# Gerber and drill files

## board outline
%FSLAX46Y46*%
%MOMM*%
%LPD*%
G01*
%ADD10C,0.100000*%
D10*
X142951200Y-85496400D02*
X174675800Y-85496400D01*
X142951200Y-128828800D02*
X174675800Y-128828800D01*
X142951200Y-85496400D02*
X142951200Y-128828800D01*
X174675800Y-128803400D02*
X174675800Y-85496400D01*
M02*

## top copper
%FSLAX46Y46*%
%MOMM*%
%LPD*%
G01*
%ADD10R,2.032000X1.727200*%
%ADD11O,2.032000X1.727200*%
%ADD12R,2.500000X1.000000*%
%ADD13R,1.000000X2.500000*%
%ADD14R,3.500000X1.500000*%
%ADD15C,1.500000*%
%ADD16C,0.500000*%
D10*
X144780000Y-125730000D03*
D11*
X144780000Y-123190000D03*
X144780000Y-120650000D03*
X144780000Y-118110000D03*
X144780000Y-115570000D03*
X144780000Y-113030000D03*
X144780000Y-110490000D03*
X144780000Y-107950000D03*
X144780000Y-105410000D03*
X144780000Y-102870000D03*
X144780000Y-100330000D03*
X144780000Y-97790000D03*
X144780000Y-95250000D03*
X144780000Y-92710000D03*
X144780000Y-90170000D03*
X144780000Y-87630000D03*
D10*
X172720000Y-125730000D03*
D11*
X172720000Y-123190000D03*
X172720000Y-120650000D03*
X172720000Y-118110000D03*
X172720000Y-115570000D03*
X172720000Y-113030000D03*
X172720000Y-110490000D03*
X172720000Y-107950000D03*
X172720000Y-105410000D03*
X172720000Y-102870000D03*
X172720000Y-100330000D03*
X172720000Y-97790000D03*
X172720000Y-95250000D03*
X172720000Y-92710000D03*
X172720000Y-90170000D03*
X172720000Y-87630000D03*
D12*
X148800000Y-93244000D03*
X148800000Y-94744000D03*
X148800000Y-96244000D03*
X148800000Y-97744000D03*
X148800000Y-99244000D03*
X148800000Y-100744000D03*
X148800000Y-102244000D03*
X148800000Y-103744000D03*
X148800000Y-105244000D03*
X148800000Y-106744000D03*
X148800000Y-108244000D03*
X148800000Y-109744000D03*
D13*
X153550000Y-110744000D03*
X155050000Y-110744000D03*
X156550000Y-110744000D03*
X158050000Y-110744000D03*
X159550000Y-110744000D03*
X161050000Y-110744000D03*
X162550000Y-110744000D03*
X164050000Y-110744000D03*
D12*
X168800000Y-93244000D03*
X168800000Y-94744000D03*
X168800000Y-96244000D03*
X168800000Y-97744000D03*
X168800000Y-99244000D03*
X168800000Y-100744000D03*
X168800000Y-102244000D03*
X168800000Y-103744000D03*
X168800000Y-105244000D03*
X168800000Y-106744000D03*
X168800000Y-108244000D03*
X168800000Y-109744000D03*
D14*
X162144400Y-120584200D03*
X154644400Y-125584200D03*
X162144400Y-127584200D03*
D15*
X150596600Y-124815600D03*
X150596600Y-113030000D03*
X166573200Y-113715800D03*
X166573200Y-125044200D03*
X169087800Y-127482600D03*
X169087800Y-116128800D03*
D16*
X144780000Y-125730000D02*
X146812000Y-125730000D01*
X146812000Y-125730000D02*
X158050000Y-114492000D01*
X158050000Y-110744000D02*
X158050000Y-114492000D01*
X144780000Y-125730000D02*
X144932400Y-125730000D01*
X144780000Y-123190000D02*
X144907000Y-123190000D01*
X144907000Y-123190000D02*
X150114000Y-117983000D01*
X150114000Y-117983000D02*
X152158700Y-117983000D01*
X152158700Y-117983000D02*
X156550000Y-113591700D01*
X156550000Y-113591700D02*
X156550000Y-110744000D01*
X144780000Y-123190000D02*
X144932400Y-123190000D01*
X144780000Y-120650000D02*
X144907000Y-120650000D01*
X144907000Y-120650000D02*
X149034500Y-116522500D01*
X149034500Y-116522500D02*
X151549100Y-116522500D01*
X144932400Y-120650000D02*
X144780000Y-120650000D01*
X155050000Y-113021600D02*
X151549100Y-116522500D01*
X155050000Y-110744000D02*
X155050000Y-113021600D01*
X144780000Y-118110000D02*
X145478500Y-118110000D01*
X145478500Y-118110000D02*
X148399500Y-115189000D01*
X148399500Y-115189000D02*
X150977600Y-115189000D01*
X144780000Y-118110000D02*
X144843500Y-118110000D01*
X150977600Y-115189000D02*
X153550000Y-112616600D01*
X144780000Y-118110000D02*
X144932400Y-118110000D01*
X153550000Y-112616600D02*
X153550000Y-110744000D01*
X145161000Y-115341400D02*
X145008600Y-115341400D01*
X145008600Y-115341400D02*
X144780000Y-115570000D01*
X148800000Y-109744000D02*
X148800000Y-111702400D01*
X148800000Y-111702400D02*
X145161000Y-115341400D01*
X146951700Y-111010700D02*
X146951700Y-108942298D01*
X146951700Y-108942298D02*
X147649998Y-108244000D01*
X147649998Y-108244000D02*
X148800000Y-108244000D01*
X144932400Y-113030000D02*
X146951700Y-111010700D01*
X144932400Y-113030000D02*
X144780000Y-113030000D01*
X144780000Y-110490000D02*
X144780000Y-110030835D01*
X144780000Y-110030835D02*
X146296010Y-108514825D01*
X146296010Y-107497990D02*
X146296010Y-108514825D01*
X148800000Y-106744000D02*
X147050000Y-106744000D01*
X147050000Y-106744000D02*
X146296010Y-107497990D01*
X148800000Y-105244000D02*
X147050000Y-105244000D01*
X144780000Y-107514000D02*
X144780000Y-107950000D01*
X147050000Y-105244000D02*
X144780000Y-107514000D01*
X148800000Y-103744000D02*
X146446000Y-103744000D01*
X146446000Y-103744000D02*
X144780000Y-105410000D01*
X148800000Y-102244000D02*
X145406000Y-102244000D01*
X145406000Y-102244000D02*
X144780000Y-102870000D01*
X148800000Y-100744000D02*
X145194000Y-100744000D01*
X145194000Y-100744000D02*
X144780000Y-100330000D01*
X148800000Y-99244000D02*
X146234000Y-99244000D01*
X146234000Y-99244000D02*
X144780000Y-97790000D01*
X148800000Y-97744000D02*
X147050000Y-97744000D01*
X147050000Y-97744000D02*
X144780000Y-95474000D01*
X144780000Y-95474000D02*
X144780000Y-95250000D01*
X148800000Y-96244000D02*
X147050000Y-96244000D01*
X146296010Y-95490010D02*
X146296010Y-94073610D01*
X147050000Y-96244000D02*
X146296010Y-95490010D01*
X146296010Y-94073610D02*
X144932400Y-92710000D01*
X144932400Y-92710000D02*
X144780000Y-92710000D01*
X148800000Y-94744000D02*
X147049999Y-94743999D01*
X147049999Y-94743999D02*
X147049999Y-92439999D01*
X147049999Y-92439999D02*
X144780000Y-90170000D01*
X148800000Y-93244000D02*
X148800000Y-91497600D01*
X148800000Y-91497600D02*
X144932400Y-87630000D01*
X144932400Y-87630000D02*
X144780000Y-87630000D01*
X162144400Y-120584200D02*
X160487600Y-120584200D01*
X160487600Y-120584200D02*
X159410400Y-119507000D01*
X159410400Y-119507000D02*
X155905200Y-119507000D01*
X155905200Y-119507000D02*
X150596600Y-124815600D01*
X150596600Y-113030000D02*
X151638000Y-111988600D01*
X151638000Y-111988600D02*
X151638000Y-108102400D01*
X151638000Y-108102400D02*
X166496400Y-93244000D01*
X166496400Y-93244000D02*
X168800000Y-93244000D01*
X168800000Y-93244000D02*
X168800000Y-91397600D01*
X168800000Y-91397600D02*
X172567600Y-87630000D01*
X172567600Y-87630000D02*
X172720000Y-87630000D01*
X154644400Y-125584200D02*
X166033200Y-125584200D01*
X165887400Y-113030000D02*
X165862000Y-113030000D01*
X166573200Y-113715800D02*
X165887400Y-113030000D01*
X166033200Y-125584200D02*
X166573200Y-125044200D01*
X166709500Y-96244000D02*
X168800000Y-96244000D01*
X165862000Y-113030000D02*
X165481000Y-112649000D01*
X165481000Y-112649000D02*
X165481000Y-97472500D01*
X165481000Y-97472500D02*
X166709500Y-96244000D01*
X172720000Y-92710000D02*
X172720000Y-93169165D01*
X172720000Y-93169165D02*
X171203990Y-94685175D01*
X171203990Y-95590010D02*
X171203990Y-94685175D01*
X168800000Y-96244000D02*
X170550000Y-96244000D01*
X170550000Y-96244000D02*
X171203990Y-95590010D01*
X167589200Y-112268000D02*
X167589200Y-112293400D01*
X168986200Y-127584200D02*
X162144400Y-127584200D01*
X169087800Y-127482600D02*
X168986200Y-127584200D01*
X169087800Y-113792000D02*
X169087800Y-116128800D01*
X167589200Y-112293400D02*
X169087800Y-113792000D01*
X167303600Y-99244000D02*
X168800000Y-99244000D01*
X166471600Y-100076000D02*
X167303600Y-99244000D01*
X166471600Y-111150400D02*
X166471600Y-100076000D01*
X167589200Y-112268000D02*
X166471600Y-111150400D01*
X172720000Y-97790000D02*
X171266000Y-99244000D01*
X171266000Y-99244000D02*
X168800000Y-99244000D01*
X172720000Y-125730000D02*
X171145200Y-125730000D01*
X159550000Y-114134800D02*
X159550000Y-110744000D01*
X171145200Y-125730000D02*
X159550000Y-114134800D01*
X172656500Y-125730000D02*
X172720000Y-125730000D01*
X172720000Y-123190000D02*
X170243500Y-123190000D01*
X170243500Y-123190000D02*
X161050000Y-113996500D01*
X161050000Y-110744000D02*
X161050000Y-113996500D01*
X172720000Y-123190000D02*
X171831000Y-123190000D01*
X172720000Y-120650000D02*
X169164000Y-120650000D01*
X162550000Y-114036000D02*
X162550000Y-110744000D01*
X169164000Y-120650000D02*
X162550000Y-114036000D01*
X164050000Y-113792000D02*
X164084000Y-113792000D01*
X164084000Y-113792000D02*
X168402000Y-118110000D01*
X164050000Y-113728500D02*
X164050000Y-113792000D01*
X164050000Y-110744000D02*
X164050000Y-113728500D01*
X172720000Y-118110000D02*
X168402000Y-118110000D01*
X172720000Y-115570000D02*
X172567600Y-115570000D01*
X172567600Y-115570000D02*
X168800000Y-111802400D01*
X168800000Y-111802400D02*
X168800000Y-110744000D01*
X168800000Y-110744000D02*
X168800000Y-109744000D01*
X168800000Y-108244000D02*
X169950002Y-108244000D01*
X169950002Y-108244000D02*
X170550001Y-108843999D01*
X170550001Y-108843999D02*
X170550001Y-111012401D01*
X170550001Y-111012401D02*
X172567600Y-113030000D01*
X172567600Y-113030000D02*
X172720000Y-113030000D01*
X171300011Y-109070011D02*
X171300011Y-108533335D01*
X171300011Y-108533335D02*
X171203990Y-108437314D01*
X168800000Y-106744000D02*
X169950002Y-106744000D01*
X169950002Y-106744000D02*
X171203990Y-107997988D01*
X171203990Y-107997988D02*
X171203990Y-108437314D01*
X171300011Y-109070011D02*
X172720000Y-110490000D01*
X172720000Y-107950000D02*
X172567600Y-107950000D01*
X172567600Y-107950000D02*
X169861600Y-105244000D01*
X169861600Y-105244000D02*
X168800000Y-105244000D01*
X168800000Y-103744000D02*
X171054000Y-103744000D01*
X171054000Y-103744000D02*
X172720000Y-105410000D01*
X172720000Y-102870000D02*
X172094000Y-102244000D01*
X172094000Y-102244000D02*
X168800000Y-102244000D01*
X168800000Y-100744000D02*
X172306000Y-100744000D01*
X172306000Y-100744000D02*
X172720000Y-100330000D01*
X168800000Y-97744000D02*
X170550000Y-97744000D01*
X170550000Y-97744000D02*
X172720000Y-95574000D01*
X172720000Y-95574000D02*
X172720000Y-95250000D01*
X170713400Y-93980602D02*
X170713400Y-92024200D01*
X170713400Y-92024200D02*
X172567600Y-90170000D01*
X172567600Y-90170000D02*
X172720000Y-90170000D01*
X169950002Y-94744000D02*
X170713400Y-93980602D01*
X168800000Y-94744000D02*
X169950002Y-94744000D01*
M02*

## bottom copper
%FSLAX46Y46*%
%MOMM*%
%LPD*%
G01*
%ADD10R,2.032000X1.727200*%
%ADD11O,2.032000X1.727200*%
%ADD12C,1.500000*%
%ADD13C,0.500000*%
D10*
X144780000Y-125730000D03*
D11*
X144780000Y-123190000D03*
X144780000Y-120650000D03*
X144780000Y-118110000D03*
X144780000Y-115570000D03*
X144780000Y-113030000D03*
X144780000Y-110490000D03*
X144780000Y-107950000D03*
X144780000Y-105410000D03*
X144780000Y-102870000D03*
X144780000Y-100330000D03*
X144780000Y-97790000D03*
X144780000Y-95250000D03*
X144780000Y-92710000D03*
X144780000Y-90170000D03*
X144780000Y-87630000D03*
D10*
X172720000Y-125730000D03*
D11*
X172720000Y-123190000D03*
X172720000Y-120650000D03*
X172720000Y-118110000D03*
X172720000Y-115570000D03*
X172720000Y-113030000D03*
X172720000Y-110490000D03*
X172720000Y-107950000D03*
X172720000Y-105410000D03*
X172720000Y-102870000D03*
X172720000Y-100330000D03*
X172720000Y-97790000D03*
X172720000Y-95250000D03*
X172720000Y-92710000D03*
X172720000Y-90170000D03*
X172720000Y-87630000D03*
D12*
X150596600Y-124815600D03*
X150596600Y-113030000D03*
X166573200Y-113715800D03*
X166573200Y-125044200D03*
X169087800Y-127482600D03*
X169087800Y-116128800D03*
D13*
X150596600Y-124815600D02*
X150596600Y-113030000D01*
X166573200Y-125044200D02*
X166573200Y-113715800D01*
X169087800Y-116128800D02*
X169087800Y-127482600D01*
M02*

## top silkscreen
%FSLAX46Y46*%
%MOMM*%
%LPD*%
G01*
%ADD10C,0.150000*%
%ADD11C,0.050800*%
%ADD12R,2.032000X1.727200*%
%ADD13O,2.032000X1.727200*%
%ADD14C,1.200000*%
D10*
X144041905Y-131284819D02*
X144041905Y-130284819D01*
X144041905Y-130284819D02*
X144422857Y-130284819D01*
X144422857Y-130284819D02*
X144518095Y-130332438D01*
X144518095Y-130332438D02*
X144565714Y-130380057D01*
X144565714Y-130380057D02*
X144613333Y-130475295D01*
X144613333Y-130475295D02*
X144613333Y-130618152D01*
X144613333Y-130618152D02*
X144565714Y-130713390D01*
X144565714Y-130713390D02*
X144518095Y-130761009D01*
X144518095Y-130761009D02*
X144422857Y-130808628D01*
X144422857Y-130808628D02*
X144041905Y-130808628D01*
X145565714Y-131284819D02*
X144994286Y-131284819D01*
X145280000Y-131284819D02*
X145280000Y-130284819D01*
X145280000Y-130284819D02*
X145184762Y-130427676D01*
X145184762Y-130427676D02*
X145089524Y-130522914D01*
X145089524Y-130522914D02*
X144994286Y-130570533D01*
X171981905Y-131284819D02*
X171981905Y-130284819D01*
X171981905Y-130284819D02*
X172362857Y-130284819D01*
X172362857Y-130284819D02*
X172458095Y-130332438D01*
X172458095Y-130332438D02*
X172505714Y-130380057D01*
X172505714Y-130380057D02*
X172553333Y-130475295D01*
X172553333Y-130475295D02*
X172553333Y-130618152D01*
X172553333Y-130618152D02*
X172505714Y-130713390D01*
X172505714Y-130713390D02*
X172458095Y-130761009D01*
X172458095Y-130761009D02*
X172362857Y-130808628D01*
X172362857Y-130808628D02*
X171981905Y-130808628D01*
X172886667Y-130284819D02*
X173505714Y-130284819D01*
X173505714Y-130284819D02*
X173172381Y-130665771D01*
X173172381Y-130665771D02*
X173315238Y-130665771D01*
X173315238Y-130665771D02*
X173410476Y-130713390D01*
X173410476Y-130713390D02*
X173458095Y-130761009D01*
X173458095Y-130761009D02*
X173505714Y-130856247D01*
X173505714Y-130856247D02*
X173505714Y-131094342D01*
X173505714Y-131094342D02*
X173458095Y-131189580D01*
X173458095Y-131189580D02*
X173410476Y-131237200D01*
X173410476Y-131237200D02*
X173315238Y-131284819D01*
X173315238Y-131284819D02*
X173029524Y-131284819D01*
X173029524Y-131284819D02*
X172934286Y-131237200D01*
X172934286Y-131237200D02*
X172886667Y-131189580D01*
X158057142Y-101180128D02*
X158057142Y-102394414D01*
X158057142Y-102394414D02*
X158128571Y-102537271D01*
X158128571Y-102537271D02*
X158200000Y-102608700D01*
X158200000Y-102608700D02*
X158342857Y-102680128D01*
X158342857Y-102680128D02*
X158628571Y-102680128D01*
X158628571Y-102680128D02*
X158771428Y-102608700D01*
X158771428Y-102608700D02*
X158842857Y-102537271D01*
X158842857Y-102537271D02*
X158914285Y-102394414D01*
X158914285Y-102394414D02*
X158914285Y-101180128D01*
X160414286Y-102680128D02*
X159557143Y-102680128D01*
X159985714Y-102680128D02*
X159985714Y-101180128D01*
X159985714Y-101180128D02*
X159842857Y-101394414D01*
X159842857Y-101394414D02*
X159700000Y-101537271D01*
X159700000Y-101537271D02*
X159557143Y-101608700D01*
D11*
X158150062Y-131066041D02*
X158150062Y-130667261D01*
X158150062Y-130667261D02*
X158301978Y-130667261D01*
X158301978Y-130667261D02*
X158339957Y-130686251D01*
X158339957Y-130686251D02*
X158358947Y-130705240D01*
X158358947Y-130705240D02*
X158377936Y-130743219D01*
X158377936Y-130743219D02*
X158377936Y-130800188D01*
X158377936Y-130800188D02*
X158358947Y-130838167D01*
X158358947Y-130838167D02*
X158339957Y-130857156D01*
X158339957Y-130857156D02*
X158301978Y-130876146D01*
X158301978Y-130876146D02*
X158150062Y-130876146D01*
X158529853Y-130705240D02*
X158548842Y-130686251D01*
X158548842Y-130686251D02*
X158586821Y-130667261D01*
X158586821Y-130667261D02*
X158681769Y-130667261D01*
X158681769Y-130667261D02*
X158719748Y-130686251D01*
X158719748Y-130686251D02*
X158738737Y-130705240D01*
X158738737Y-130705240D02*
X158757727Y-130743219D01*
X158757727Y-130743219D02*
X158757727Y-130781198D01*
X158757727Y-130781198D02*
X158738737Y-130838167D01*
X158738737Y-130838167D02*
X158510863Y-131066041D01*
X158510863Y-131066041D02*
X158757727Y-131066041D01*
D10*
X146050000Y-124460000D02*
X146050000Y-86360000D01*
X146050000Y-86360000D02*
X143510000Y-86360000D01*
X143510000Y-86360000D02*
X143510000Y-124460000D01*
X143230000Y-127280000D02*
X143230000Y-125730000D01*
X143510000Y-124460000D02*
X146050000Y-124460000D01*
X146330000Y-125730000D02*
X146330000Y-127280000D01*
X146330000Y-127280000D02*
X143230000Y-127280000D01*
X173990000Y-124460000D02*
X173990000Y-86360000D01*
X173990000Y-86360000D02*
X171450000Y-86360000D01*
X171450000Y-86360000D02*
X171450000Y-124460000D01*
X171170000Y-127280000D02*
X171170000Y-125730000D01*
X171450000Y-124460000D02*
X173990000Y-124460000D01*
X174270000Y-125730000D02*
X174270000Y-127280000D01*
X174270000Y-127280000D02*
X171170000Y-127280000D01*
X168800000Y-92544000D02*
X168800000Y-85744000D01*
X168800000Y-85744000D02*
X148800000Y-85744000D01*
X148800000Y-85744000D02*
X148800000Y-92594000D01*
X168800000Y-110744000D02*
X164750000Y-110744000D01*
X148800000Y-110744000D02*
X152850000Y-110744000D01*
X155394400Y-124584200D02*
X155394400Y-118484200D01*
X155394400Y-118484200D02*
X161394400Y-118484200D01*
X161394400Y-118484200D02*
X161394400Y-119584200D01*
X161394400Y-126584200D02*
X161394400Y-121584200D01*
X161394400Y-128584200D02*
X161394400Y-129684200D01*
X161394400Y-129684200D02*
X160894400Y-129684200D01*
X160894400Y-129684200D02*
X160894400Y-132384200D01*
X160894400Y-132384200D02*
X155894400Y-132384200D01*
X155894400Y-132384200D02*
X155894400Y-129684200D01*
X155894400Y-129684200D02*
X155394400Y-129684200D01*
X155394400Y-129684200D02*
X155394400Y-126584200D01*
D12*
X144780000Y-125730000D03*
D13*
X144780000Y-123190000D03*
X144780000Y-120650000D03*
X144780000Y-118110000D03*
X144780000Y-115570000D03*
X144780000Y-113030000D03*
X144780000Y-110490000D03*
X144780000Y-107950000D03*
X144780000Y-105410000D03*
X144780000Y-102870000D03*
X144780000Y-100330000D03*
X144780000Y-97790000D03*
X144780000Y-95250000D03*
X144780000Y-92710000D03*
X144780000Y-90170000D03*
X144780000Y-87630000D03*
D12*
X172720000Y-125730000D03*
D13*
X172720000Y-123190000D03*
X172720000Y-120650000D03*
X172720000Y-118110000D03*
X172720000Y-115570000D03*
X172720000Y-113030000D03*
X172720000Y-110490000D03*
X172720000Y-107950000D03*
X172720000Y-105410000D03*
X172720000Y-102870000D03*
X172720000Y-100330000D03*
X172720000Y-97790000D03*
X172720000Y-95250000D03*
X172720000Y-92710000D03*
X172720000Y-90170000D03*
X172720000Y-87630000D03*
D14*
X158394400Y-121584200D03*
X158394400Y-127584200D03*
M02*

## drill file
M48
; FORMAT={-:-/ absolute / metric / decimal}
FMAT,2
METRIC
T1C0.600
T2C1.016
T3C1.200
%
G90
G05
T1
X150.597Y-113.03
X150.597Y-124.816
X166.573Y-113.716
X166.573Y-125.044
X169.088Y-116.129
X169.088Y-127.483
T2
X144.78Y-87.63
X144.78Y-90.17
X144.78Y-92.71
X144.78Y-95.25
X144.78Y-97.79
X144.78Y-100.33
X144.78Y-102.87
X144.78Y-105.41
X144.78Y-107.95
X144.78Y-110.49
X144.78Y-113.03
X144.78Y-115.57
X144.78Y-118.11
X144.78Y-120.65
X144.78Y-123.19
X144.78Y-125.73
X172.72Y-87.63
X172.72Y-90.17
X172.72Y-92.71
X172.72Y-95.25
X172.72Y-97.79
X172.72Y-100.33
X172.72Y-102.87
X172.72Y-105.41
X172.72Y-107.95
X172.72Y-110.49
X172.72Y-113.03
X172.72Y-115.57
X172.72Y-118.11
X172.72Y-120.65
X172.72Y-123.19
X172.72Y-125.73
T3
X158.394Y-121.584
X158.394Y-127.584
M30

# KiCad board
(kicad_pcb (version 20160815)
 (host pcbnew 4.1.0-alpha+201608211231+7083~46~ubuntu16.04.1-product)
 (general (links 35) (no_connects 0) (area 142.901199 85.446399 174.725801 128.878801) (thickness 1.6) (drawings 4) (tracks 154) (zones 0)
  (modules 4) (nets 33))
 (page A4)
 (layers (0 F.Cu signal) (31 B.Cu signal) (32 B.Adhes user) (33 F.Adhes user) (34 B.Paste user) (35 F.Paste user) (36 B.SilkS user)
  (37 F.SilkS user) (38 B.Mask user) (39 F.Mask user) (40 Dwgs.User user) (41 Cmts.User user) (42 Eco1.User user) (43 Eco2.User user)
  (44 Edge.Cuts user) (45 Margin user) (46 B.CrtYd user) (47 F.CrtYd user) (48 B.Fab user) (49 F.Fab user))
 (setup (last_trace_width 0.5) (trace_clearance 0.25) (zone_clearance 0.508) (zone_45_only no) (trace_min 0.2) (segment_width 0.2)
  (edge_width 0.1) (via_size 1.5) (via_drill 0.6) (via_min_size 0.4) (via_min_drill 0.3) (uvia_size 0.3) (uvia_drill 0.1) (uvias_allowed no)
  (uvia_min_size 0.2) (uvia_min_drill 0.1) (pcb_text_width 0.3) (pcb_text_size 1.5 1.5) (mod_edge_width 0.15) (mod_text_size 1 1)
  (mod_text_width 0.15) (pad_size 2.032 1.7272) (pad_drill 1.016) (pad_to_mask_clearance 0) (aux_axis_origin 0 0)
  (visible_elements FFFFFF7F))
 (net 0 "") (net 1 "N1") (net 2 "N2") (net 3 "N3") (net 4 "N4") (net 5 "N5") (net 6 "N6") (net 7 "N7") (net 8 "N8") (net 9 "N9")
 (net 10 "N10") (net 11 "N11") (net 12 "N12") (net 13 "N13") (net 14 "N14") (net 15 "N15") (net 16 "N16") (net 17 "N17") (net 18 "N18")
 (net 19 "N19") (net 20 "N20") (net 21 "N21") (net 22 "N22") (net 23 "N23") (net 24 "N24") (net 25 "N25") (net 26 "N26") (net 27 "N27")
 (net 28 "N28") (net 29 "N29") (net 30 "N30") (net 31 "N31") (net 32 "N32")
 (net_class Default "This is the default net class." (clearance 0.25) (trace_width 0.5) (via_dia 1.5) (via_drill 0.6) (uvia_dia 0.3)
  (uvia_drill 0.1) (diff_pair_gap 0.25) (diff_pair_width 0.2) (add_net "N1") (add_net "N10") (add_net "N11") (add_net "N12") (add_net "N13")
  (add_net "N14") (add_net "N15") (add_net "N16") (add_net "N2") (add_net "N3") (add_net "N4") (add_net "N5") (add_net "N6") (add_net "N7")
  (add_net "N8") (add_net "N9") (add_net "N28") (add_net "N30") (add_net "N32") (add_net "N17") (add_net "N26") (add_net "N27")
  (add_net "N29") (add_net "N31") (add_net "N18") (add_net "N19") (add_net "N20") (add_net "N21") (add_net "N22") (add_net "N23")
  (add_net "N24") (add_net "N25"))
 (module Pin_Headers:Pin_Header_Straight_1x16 (layer F.Cu) (at 144.78 125.73 180)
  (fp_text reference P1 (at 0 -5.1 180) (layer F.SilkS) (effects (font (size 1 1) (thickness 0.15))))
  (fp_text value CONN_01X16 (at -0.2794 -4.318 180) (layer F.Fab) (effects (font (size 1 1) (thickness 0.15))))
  (fp_line (start -1.27 1.27) (end -1.27 39.37) (layer F.SilkS) (width 0.15))
  (fp_line (start -1.27 39.37) (end 1.27 39.37) (layer F.SilkS) (width 0.15))
  (fp_line (start 1.27 39.37) (end 1.27 1.27) (layer F.SilkS) (width 0.15))
  (fp_line (start 1.55 -1.55) (end 1.55 0) (layer F.SilkS) (width 0.15))
  (fp_line (start 1.27 1.27) (end -1.27 1.27) (layer F.SilkS) (width 0.15))
  (fp_line (start -1.55 0) (end -1.55 -1.55) (layer F.SilkS) (width 0.15))
  (fp_line (start -1.55 -1.55) (end 1.55 -1.55) (layer F.SilkS) (width 0.15))
  (pad 1 thru_hole rect (at 0 0 180) (size 2.032 1.7272) (drill 1.016) (layers *.Cu *.Mask F.SilkS) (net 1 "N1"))
  (pad 2 thru_hole oval (at 0 2.54 180) (size 2.032 1.7272) (drill 1.016) (layers *.Cu *.Mask F.SilkS) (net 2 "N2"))
  (pad 3 thru_hole oval (at 0 5.08 180) (size 2.032 1.7272) (drill 1.016) (layers *.Cu *.Mask F.SilkS) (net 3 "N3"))
  (pad 4 thru_hole oval (at 0 7.62 180) (size 2.032 1.7272) (drill 1.016) (layers *.Cu *.Mask F.SilkS) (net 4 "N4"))
  (pad 5 thru_hole oval (at 0 10.16 180) (size 2.032 1.7272) (drill 1.016) (layers *.Cu *.Mask F.SilkS) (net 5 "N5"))
  (pad 6 thru_hole oval (at 0 12.7 180) (size 2.032 1.7272) (drill 1.016) (layers *.Cu *.Mask F.SilkS) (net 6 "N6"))
  (pad 7 thru_hole oval (at 0 15.24 180) (size 2.032 1.7272) (drill 1.016) (layers *.Cu *.Mask F.SilkS) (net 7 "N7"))
  (pad 8 thru_hole oval (at 0 17.78 180) (size 2.032 1.7272) (drill 1.016) (layers *.Cu *.Mask F.SilkS) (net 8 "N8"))
  (pad 9 thru_hole oval (at 0 20.32 180) (size 2.032 1.7272) (drill 1.016) (layers *.Cu *.Mask F.SilkS) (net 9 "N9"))
  (pad 10 thru_hole oval (at 0 22.86 180) (size 2.032 1.7272) (drill 1.016) (layers *.Cu *.Mask F.SilkS) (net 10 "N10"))
  (pad 11 thru_hole oval (at 0 25.4 180) (size 2.032 1.7272) (drill 1.016) (layers *.Cu *.Mask F.SilkS) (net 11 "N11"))
  (pad 12 thru_hole oval (at 0 27.94 180) (size 2.032 1.7272) (drill 1.016) (layers *.Cu *.Mask F.SilkS) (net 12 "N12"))
  (pad 13 thru_hole oval (at 0 30.48 180) (size 2.032 1.7272) (drill 1.016) (layers *.Cu *.Mask F.SilkS) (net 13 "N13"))
  (pad 14 thru_hole oval (at 0 33.02 180) (size 2.032 1.7272) (drill 1.016) (layers *.Cu *.Mask F.SilkS) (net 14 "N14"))
  (pad 15 thru_hole oval (at 0 35.56 180) (size 2.032 1.7272) (drill 1.016) (layers *.Cu *.Mask F.SilkS) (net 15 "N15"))
  (pad 16 thru_hole oval (at 0 38.1 180) (size 2.032 1.7272) (drill 1.016) (layers *.Cu *.Mask F.SilkS) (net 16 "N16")))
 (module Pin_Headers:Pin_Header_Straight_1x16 (layer F.Cu) (at 172.72 125.73 180)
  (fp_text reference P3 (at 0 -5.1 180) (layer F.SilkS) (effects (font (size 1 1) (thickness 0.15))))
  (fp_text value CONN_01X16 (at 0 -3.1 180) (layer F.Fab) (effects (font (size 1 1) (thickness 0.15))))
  (fp_line (start -1.27 1.27) (end -1.27 39.37) (layer F.SilkS) (width 0.15))
  (fp_line (start -1.27 39.37) (end 1.27 39.37) (layer F.SilkS) (width 0.15))
  (fp_line (start 1.27 39.37) (end 1.27 1.27) (layer F.SilkS) (width 0.15))
  (fp_line (start 1.55 -1.55) (end 1.55 0) (layer F.SilkS) (width 0.15))
  (fp_line (start 1.27 1.27) (end -1.27 1.27) (layer F.SilkS) (width 0.15))
  (fp_line (start -1.55 0) (end -1.55 -1.55) (layer F.SilkS) (width 0.15))
  (fp_line (start -1.55 -1.55) (end 1.55 -1.55) (layer F.SilkS) (width 0.15))
  (pad 1 thru_hole rect (at 0 0 180) (size 2.032 1.7272) (drill 1.016) (layers *.Cu *.Mask F.SilkS) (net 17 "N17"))
  (pad 2 thru_hole oval (at 0 2.54 180) (size 2.032 1.7272) (drill 1.016) (layers *.Cu *.Mask F.SilkS) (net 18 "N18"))
  (pad 3 thru_hole oval (at 0 5.08 180) (size 2.032 1.7272) (drill 1.016) (layers *.Cu *.Mask F.SilkS) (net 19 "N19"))
  (pad 4 thru_hole oval (at 0 7.62 180) (size 2.032 1.7272) (drill 1.016) (layers *.Cu *.Mask F.SilkS) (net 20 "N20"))
  (pad 5 thru_hole oval (at 0 10.16 180) (size 2.032 1.7272) (drill 1.016) (layers *.Cu *.Mask F.SilkS) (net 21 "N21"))
  (pad 6 thru_hole oval (at 0 12.7 180) (size 2.032 1.7272) (drill 1.016) (layers *.Cu *.Mask F.SilkS) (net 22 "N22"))
  (pad 7 thru_hole oval (at 0 15.24 180) (size 2.032 1.7272) (drill 1.016) (layers *.Cu *.Mask F.SilkS) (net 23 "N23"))
  (pad 8 thru_hole oval (at 0 17.78 180) (size 2.032 1.7272) (drill 1.016) (layers *.Cu *.Mask F.SilkS) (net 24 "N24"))
  (pad 9 thru_hole oval (at 0 20.32 180) (size 2.032 1.7272) (drill 1.016) (layers *.Cu *.Mask F.SilkS) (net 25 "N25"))
  (pad 10 thru_hole oval (at 0 22.86 180) (size 2.032 1.7272) (drill 1.016) (layers *.Cu *.Mask F.SilkS) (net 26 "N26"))
  (pad 11 thru_hole oval (at 0 25.4 180) (size 2.032 1.7272) (drill 1.016) (layers *.Cu *.Mask F.SilkS) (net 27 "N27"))
  (pad 12 thru_hole oval (at 0 27.94 180) (size 2.032 1.7272) (drill 1.016) (layers *.Cu *.Mask F.SilkS) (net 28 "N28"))
  (pad 13 thru_hole oval (at 0 30.48 180) (size 2.032 1.7272) (drill 1.016) (layers *.Cu *.Mask F.SilkS) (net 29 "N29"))
  (pad 14 thru_hole oval (at 0 33.02 180) (size 2.032 1.7272) (drill 1.016) (layers *.Cu *.Mask F.SilkS) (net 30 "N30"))
  (pad 15 thru_hole oval (at 0 35.56 180) (size 2.032 1.7272) (drill 1.016) (layers *.Cu *.Mask F.SilkS) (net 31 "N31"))
  (pad 16 thru_hole oval (at 0 38.1 180) (size 2.032 1.7272) (drill 1.016) (layers *.Cu *.Mask F.SilkS) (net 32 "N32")))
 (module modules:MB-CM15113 (layer F.Cu) (at 148.8 110.744)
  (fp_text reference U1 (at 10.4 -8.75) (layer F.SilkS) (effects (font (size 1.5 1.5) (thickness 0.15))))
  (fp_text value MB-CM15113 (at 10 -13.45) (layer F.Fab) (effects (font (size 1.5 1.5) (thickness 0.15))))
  (fp_line (start 20 -18.2) (end 20 -25) (layer F.SilkS) (width 0.15))
  (fp_line (start 20 -25) (end 0 -25) (layer F.SilkS) (width 0.15))
  (fp_line (start 0 -25) (end 0 -18.15) (layer F.SilkS) (width 0.15))
  (fp_line (start 20 0) (end 15.95 0) (layer F.SilkS) (width 0.15))
  (fp_line (start 0 0) (end 4.05 0) (layer F.SilkS) (width 0.15))
  (pad 1 smd rect (at 0 -17.5) (size 2.5 1) (layers F.Cu F.Paste F.Mask) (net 16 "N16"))
  (pad 2 smd rect (at 0 -16) (size 2.5 1) (layers F.Cu F.Paste F.Mask) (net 15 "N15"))
  (pad 3 smd rect (at 0 -14.5) (size 2.5 1) (layers F.Cu F.Paste F.Mask) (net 14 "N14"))
  (pad 4 smd rect (at 0 -13) (size 2.5 1) (layers F.Cu F.Paste F.Mask) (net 13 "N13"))
  (pad 5 smd rect (at 0 -11.5) (size 2.5 1) (layers F.Cu F.Paste F.Mask) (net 12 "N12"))
  (pad 6 smd rect (at 0 -10) (size 2.5 1) (layers F.Cu F.Paste F.Mask) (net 11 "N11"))
  (pad 7 smd rect (at 0 -8.5) (size 2.5 1) (layers F.Cu F.Paste F.Mask) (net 10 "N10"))
  (pad 8 smd rect (at 0 -7) (size 2.5 1) (layers F.Cu F.Paste F.Mask) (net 9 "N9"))
  (pad 9 smd rect (at 0 -5.5) (size 2.5 1) (layers F.Cu F.Paste F.Mask) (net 8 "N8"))
  (pad 10 smd rect (at 0 -4) (size 2.5 1) (layers F.Cu F.Paste F.Mask) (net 7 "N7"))
  (pad 11 smd rect (at 0 -2.5) (size 2.5 1) (layers F.Cu F.Paste F.Mask) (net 6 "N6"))
  (pad 12 smd rect (at 0 -1) (size 2.5 1) (layers F.Cu F.Paste F.Mask) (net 5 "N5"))
  (pad 13 smd rect (at 4.75 0) (size 1 2.5) (layers F.Cu F.Paste F.Mask) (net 4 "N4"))
  (pad 14 smd rect (at 6.25 0) (size 1 2.5) (layers F.Cu F.Paste F.Mask) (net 3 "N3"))
  (pad 15 smd rect (at 7.75 0) (size 1 2.5) (layers F.Cu F.Paste F.Mask) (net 2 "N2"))
  (pad 16 smd rect (at 9.25 0) (size 1 2.5) (layers F.Cu F.Paste F.Mask) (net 1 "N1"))
  (pad 17 smd rect (at 10.75 0) (size 1 2.5) (layers F.Cu F.Paste F.Mask) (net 17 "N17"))
  (pad 18 smd rect (at 12.25 0) (size 1 2.5) (layers F.Cu F.Paste F.Mask) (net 18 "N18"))
  (pad 19 smd rect (at 13.75 0) (size 1 2.5) (layers F.Cu F.Paste F.Mask) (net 19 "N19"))
  (pad 20 smd rect (at 15.25 0) (size 1 2.5) (layers F.Cu F.Paste F.Mask) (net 20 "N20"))
  (pad 32 smd rect (at 20 -17.5) (size 2.5 1) (layers F.Cu F.Paste F.Mask) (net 32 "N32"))
  (pad 31 smd rect (at 20 -16) (size 2.5 1) (layers F.Cu F.Paste F.Mask) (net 31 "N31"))
  (pad 30 smd rect (at 20 -14.5) (size 2.5 1) (layers F.Cu F.Paste F.Mask) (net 30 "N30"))
  (pad 29 smd rect (at 20 -13) (size 2.5 1) (layers F.Cu F.Paste F.Mask) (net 29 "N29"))
  (pad 28 smd rect (at 20 -11.5) (size 2.5 1) (layers F.Cu F.Paste F.Mask) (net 28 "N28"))
  (pad 27 smd rect (at 20 -10) (size 2.5 1) (layers F.Cu F.Paste F.Mask) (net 27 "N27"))
  (pad 26 smd rect (at 20 -8.5) (size 2.5 1) (layers F.Cu F.Paste F.Mask) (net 26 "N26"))
  (pad 25 smd rect (at 20 -7) (size 2.5 1) (layers F.Cu F.Paste F.Mask) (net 25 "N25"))
  (pad 24 smd rect (at 20 -5.5) (size 2.5 1) (layers F.Cu F.Paste F.Mask) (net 24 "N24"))
  (pad 23 smd rect (at 20 -4) (size 2.5 1) (layers F.Cu F.Paste F.Mask) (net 23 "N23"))
  (pad 22 smd rect (at 20 -2.5) (size 2.5 1) (layers F.Cu F.Paste F.Mask) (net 22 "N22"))
  (pad 21 smd rect (at 20 -1) (size 2.5 1) (layers F.Cu F.Paste F.Mask) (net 21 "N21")))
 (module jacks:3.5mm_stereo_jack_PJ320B (layer F.Cu) (at 158.3944 127.5842 180)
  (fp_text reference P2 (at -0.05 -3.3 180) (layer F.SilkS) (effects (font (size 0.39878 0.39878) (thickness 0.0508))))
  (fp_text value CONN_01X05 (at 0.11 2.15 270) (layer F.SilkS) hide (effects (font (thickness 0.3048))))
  (fp_line (start 3 3) (end 3 9.1) (layer F.SilkS) (width 0.15))
  (fp_line (start 3 9.1) (end -3 9.1) (layer F.SilkS) (width 0.15))
  (fp_line (start -3 9.1) (end -3 8) (layer F.SilkS) (width 0.15))
  (fp_line (start -3 1) (end -3 6) (layer F.SilkS) (width 0.15))
  (fp_line (start -3 -1) (end -3 -2.1) (layer F.SilkS) (width 0.15))
  (fp_line (start -3 -2.1) (end -2.5 -2.1) (layer F.SilkS) (width 0.15))
  (fp_line (start -2.5 -2.1) (end -2.5 -4.8) (layer F.SilkS) (width 0.15))
  (fp_line (start -2.5 -4.8) (end 2.5 -4.8) (layer F.SilkS) (width 0.15))
  (fp_line (start 2.5 -4.8) (end 2.5 -2.1) (layer F.SilkS) (width 0.15))
  (fp_line (start 2.5 -2.1) (end 3 -2.1) (layer F.SilkS) (width 0.15))
  (fp_line (start 3 -2.1) (end 3 1) (layer F.SilkS) (width 0.15))
  (pad "" np_thru_hole circle (at 0 6 180) (size 1.2 1.2) (drill 1.2) (layers *.Cu *.Mask F.SilkS))
  (pad 5 smd rect (at -3.75 7 180) (size 3.5 1.5) (layers F.Cu F.Paste F.Mask) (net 32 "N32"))
  (pad 2 smd rect (at 3.75 2 180) (size 3.5 1.5) (layers F.Cu F.Paste F.Mask) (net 30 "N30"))
  (pad 1 smd rect (at -3.75 0 180) (size 3.5 1.5) (layers F.Cu F.Paste F.Mask) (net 28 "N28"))
  (pad "" np_thru_hole circle (at 0 0 180) (size 1.2 1.2) (drill 1.2) (layers *.Cu *.Mask F.SilkS)))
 (gr_line (start 142.9512 85.4964) (end 174.6758 85.4964) (angle 90) (layer Edge.Cuts) (width 0.1))
 (gr_line (start 142.9512 128.8288) (end 174.6758 128.8288) (angle 90) (layer Edge.Cuts) (width 0.1))
 (gr_line (start 142.9512 85.4964) (end 142.9512 128.8288) (angle 90) (layer Edge.Cuts) (width 0.1))
 (gr_line (start 174.6758 128.8034) (end 174.6758 85.4964) (angle 90) (layer Edge.Cuts) (width 0.1))
 (segment (start 144.78 125.73) (end 146.812 125.73) (width 0.5) (layer F.Cu) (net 1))
 (segment (start 146.812 125.73) (end 158.05 114.492) (width 0.5) (layer F.Cu) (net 1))
 (segment (start 158.05 110.744) (end 158.05 114.492) (width 0.5) (layer F.Cu) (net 1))
 (segment (start 144.78 125.73) (end 144.9324 125.73) (width 0.5) (layer F.Cu) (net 1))
 (segment (start 144.78 123.19) (end 144.907 123.19) (width 0.5) (layer F.Cu) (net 2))
 (segment (start 144.907 123.19) (end 150.114 117.983) (width 0.5) (layer F.Cu) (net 2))
 (segment (start 150.114 117.983) (end 152.1587 117.983) (width 0.5) (layer F.Cu) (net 2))
 (segment (start 152.1587 117.983) (end 156.55 113.5917) (width 0.5) (layer F.Cu) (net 2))
 (segment (start 156.55 113.5917) (end 156.55 110.744) (width 0.5) (layer F.Cu) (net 2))
 (segment (start 144.78 123.19) (end 144.9324 123.19) (width 0.5) (layer F.Cu) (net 2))
 (segment (start 144.78 120.65) (end 144.907 120.65) (width 0.5) (layer F.Cu) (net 3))
 (segment (start 144.907 120.65) (end 149.0345 116.5225) (width 0.5) (layer F.Cu) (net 3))
 (segment (start 149.0345 116.5225) (end 151.5491 116.5225) (width 0.5) (layer F.Cu) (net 3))
 (segment (start 144.9324 120.65) (end 144.78 120.65) (width 0.5) (layer F.Cu) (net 3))
 (segment (start 155.05 113.0216) (end 151.5491 116.5225) (width 0.5) (layer F.Cu) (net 3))
 (segment (start 155.05 110.744) (end 155.05 113.0216) (width 0.5) (layer F.Cu) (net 3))
 (segment (start 144.78 118.11) (end 145.4785 118.11) (width 0.5) (layer F.Cu) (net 4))
 (segment (start 145.4785 118.11) (end 148.3995 115.189) (width 0.5) (layer F.Cu) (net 4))
 (segment (start 148.3995 115.189) (end 150.9776 115.189) (width 0.5) (layer F.Cu) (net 4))
 (segment (start 144.78 118.11) (end 144.8435 118.11) (width 0.5) (layer F.Cu) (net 4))
 (segment (start 150.9776 115.189) (end 153.55 112.6166) (width 0.5) (layer F.Cu) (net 4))
 (segment (start 144.78 118.11) (end 144.9324 118.11) (width 0.5) (layer F.Cu) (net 4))
 (segment (start 153.55 112.6166) (end 153.55 110.744) (width 0.5) (layer F.Cu) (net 4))
 (segment (start 145.161 115.3414) (end 145.0086 115.3414) (width 0.5) (layer F.Cu) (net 5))
 (segment (start 145.0086 115.3414) (end 144.78 115.57) (width 0.5) (layer F.Cu) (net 5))
 (segment (start 148.8 109.744) (end 148.8 111.7024) (width 0.5) (layer F.Cu) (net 5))
 (segment (start 148.8 111.7024) (end 145.161 115.3414) (width 0.5) (layer F.Cu) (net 5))
 (segment (start 146.9517 111.0107) (end 146.9517 108.942298) (width 0.5) (layer F.Cu) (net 6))
 (segment (start 146.9517 108.942298) (end 147.649998 108.244) (width 0.5) (layer F.Cu) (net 6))
 (segment (start 147.649998 108.244) (end 148.8 108.244) (width 0.5) (layer F.Cu) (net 6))
 (segment (start 144.9324 113.03) (end 146.9517 111.0107) (width 0.5) (layer F.Cu) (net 6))
 (segment (start 144.9324 113.03) (end 144.78 113.03) (width 0.5) (layer F.Cu) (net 6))
 (segment (start 144.78 110.49) (end 144.78 110.030835) (width 0.5) (layer F.Cu) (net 7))
 (segment (start 144.78 110.030835) (end 146.29601 108.514825) (width 0.5) (layer F.Cu) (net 7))
 (segment (start 146.29601 107.49799) (end 146.29601 108.514825) (width 0.5) (layer F.Cu) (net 7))
 (segment (start 148.8 106.744) (end 147.05 106.744) (width 0.5) (layer F.Cu) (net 7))
 (segment (start 147.05 106.744) (end 146.29601 107.49799) (width 0.5) (layer F.Cu) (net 7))
 (segment (start 148.8 105.244) (end 147.05 105.244) (width 0.5) (layer F.Cu) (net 8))
 (segment (start 144.78 107.514) (end 144.78 107.95) (width 0.5) (layer F.Cu) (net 8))
 (segment (start 147.05 105.244) (end 144.78 107.514) (width 0.5) (layer F.Cu) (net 8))
 (segment (start 148.8 103.744) (end 146.446 103.744) (width 0.5) (layer F.Cu) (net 9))
 (segment (start 146.446 103.744) (end 144.78 105.41) (width 0.5) (layer F.Cu) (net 9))
 (segment (start 148.8 102.244) (end 145.406 102.244) (width 0.5) (layer F.Cu) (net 10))
 (segment (start 145.406 102.244) (end 144.78 102.87) (width 0.5) (layer F.Cu) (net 10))
 (segment (start 148.8 100.744) (end 145.194 100.744) (width 0.5) (layer F.Cu) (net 11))
 (segment (start 145.194 100.744) (end 144.78 100.33) (width 0.5) (layer F.Cu) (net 11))
 (segment (start 148.8 99.244) (end 146.234 99.244) (width 0.5) (layer F.Cu) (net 12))
 (segment (start 146.234 99.244) (end 144.78 97.79) (width 0.5) (layer F.Cu) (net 12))
 (segment (start 148.8 97.744) (end 147.05 97.744) (width 0.5) (layer F.Cu) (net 13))
 (segment (start 147.05 97.744) (end 144.78 95.474) (width 0.5) (layer F.Cu) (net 13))
 (segment (start 144.78 95.474) (end 144.78 95.25) (width 0.5) (layer F.Cu) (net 13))
 (segment (start 148.8 96.244) (end 147.05 96.244) (width 0.5) (layer F.Cu) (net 14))
 (segment (start 146.29601 95.49001) (end 146.29601 94.07361) (width 0.5) (layer F.Cu) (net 14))
 (segment (start 147.05 96.244) (end 146.29601 95.49001) (width 0.5) (layer F.Cu) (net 14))
 (segment (start 146.29601 94.07361) (end 144.9324 92.71) (width 0.5) (layer F.Cu) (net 14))
 (segment (start 144.9324 92.71) (end 144.78 92.71) (width 0.5) (layer F.Cu) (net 14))
 (segment (start 148.8 94.744) (end 147.049999 94.743999) (width 0.5) (layer F.Cu) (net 15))
 (segment (start 147.049999 94.743999) (end 147.049999 92.439999) (width 0.5) (layer F.Cu) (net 15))
 (segment (start 147.049999 92.439999) (end 144.78 90.17) (width 0.5) (layer F.Cu) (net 15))
 (segment (start 148.8 93.244) (end 148.8 91.4976) (width 0.5) (layer F.Cu) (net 16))
 (segment (start 148.8 91.4976) (end 144.9324 87.63) (width 0.5) (layer F.Cu) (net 16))
 (segment (start 144.9324 87.63) (end 144.78 87.63) (width 0.5) (layer F.Cu) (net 16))
 (segment (start 162.1444 120.5842) (end 160.4876 120.5842) (width 0.5) (layer F.Cu) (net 32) (status C00000))
 (segment (start 160.4876 120.5842) (end 159.4104 119.507) (width 0.5) (layer F.Cu) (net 32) (status 400000))
 (segment (start 159.4104 119.507) (end 155.9052 119.507) (width 0.5) (layer F.Cu) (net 32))
 (segment (start 155.9052 119.507) (end 150.5966 124.8156) (width 0.5) (layer F.Cu) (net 32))
 (via (at 150.5966 124.8156) (size 1.5) (drill 0.6) (layers F.Cu B.Cu) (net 32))
 (segment (start 150.5966 124.8156) (end 150.5966 113.03) (width 0.5) (layer B.Cu) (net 32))
 (via (at 150.5966 113.03) (size 1.5) (drill 0.6) (layers F.Cu B.Cu) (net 32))
 (segment (start 150.5966 113.03) (end 151.638 111.9886) (width 0.5) (layer F.Cu) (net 32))
 (segment (start 151.638 111.9886) (end 151.638 108.1024) (width 0.5) (layer F.Cu) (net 32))
 (segment (start 151.638 108.1024) (end 166.4964 93.244) (width 0.5) (layer F.Cu) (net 32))
 (segment (start 166.4964 93.244) (end 168.8 93.244) (width 0.5) (layer F.Cu) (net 32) (status 800000))
 (segment (start 168.8 93.244) (end 168.8 91.3976) (width 0.5) (layer F.Cu) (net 32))
 (segment (start 168.8 91.3976) (end 172.5676 87.63) (width 0.5) (layer F.Cu) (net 32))
 (segment (start 172.5676 87.63) (end 172.72 87.63) (width 0.5) (layer F.Cu) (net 32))
 (segment (start 154.6444 125.5842) (end 166.0332 125.5842) (width 0.5) (layer F.Cu) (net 30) (status 400000))
 (segment (start 165.8874 113.03) (end 165.862 113.03) (width 0.5) (layer F.Cu) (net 30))
 (segment (start 166.5732 113.7158) (end 165.8874 113.03) (width 0.5) (layer F.Cu) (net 30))
 (via (at 166.5732 113.7158) (size 1.5) (drill 0.6) (layers F.Cu B.Cu) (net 30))
 (segment (start 166.5732 125.0442) (end 166.5732 113.7158) (width 0.5) (layer B.Cu) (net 30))
 (via (at 166.5732 125.0442) (size 1.5) (drill 0.6) (layers F.Cu B.Cu) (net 30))
 (segment (start 166.0332 125.5842) (end 166.5732 125.0442) (width 0.5) (layer F.Cu) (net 30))
 (segment (start 166.7095 96.244) (end 168.8 96.244) (width 0.5) (layer F.Cu) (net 30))
 (segment (start 165.862 113.03) (end 165.481 112.649) (width 0.5) (layer F.Cu) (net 30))
 (segment (start 165.481 112.649) (end 165.481 97.4725) (width 0.5) (layer F.Cu) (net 30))
 (segment (start 165.481 97.4725) (end 166.7095 96.244) (width 0.5) (layer F.Cu) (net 30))
 (segment (start 172.72 92.71) (end 172.72 93.169165) (width 0.5) (layer F.Cu) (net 30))
 (segment (start 172.72 93.169165) (end 171.20399 94.685175) (width 0.5) (layer F.Cu) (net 30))
 (segment (start 171.20399 95.59001) (end 171.20399 94.685175) (width 0.5) (layer F.Cu) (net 30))
 (segment (start 168.8 96.244) (end 170.55 96.244) (width 0.5) (layer F.Cu) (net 30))
 (segment (start 170.55 96.244) (end 171.20399 95.59001) (width 0.5) (layer F.Cu) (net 30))
 (segment (start 167.5892 112.268) (end 167.5892 112.2934) (width 0.5) (layer F.Cu) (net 28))
 (segment (start 168.9862 127.5842) (end 162.1444 127.5842) (width 0.5) (layer F.Cu) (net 28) (status 800000))
 (segment (start 169.0878 127.4826) (end 168.9862 127.5842) (width 0.5) (layer F.Cu) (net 28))
 (via (at 169.0878 127.4826) (size 1.5) (drill 0.6) (layers F.Cu B.Cu) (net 28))
 (segment (start 169.0878 116.1288) (end 169.0878 127.4826) (width 0.5) (layer B.Cu) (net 28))
 (via (at 169.0878 116.1288) (size 1.5) (drill 0.6) (layers F.Cu B.Cu) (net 28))
 (segment (start 169.0878 113.792) (end 169.0878 116.1288) (width 0.5) (layer F.Cu) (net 28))
 (segment (start 167.5892 112.2934) (end 169.0878 113.792) (width 0.5) (layer F.Cu) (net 28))
 (segment (start 167.3036 99.244) (end 168.8 99.244) (width 0.5) (layer F.Cu) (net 28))
 (segment (start 166.4716 100.076) (end 167.3036 99.244) (width 0.5) (layer F.Cu) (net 28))
 (segment (start 166.4716 111.1504) (end 166.4716 100.076) (width 0.5) (layer F.Cu) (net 28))
 (segment (start 167.5892 112.268) (end 166.4716 111.1504) (width 0.5) (layer F.Cu) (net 28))
 (segment (start 172.72 97.79) (end 171.266 99.244) (width 0.5) (layer F.Cu) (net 28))
 (segment (start 171.266 99.244) (end 168.8 99.244) (width 0.5) (layer F.Cu) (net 28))
 (segment (start 172.72 125.73) (end 171.1452 125.73) (width 0.5) (layer F.Cu) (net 17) (status 400000))
 (segment (start 159.55 114.1348) (end 159.55 110.744) (width 0.5) (layer F.Cu) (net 17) (status 800000))
 (segment (start 171.1452 125.73) (end 159.55 114.1348) (width 0.5) (layer F.Cu) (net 17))
 (segment (start 172.6565 125.73) (end 172.72 125.73) (width 0.5) (layer F.Cu) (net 17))
 (segment (start 172.72 123.19) (end 170.2435 123.19) (width 0.5) (layer F.Cu) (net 18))
 (segment (start 170.2435 123.19) (end 161.05 113.9965) (width 0.5) (layer F.Cu) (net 18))
 (segment (start 161.05 110.744) (end 161.05 113.9965) (width 0.5) (layer F.Cu) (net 18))
 (segment (start 172.72 123.19) (end 171.831 123.19) (width 0.5) (layer F.Cu) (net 18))
 (segment (start 172.72 120.65) (end 169.164 120.65) (width 0.5) (layer F.Cu) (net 19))
 (segment (start 162.55 114.036) (end 162.55 110.744) (width 0.5) (layer F.Cu) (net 19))
 (segment (start 169.164 120.65) (end 162.55 114.036) (width 0.5) (layer F.Cu) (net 19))
 (segment (start 164.05 113.792) (end 164.084 113.792) (width 0.5) (layer F.Cu) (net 20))
 (segment (start 164.084 113.792) (end 168.402 118.11) (width 0.5) (layer F.Cu) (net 20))
 (segment (start 164.05 113.7285) (end 164.05 113.792) (width 0.5) (layer F.Cu) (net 20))
 (segment (start 164.05 110.744) (end 164.05 113.7285) (width 0.5) (layer F.Cu) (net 20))
 (segment (start 172.72 118.11) (end 168.402 118.11) (width 0.5) (layer F.Cu) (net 20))
 (segment (start 172.72 115.57) (end 172.5676 115.57) (width 0.5) (layer F.Cu) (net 21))
 (segment (start 172.5676 115.57) (end 168.8 111.8024) (width 0.5) (layer F.Cu) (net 21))
 (segment (start 168.8 111.8024) (end 168.8 110.744) (width 0.5) (layer F.Cu) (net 21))
 (segment (start 168.8 110.744) (end 168.8 109.744) (width 0.5) (layer F.Cu) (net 21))
 (segment (start 168.8 108.244) (end 169.950002 108.244) (width 0.5) (layer F.Cu) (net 22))
 (segment (start 169.950002 108.244) (end 170.550001 108.843999) (width 0.5) (layer F.Cu) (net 22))
 (segment (start 170.550001 108.843999) (end 170.550001 111.012401) (width 0.5) (layer F.Cu) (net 22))
 (segment (start 170.550001 111.012401) (end 172.5676 113.03) (width 0.5) (layer F.Cu) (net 22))
 (segment (start 172.5676 113.03) (end 172.72 113.03) (width 0.5) (layer F.Cu) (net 22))
 (segment (start 171.300011 109.070011) (end 171.300011 108.533335) (width 0.5) (layer F.Cu) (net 23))
 (segment (start 171.300011 108.533335) (end 171.20399 108.437314) (width 0.5) (layer F.Cu) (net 23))
 (segment (start 168.8 106.744) (end 169.950002 106.744) (width 0.5) (layer F.Cu) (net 23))
 (segment (start 169.950002 106.744) (end 171.20399 107.997988) (width 0.5) (layer F.Cu) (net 23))
 (segment (start 171.20399 107.997988) (end 171.20399 108.437314) (width 0.5) (layer F.Cu) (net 23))
 (segment (start 171.300011 109.070011) (end 172.72 110.49) (width 0.5) (layer F.Cu) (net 23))
 (segment (start 172.72 107.95) (end 172.5676 107.95) (width 0.5) (layer F.Cu) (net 24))
 (segment (start 172.5676 107.95) (end 169.8616 105.244) (width 0.5) (layer F.Cu) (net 24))
 (segment (start 169.8616 105.244) (end 168.8 105.244) (width 0.5) (layer F.Cu) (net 24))
 (segment (start 168.8 103.744) (end 171.054 103.744) (width 0.5) (layer F.Cu) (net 25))
 (segment (start 171.054 103.744) (end 172.72 105.41) (width 0.5) (layer F.Cu) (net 25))
 (segment (start 172.72 102.87) (end 172.094 102.244) (width 0.5) (layer F.Cu) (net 26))
 (segment (start 172.094 102.244) (end 168.8 102.244) (width 0.5) (layer F.Cu) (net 26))
 (segment (start 168.8 100.744) (end 172.306 100.744) (width 0.5) (layer F.Cu) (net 27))
 (segment (start 172.306 100.744) (end 172.72 100.33) (width 0.5) (layer F.Cu) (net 27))
 (segment (start 168.8 97.744) (end 170.55 97.744) (width 0.5) (layer F.Cu) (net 29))
 (segment (start 170.55 97.744) (end 172.72 95.574) (width 0.5) (layer F.Cu) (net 29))
 (segment (start 172.72 95.574) (end 172.72 95.25) (width 0.5) (layer F.Cu) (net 29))
 (segment (start 170.7134 93.980602) (end 170.7134 92.0242) (width 0.5) (layer F.Cu) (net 31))
 (segment (start 170.7134 92.0242) (end 172.5676 90.17) (width 0.5) (layer F.Cu) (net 31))
 (segment (start 172.5676 90.17) (end 172.72 90.17) (width 0.5) (layer F.Cu) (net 31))
 (segment (start 169.950002 94.744) (end 170.7134 93.980602) (width 0.5) (layer F.Cu) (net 31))
 (segment (start 168.8 94.744) (end 169.950002 94.744) (width 0.5) (layer F.Cu) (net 31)))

